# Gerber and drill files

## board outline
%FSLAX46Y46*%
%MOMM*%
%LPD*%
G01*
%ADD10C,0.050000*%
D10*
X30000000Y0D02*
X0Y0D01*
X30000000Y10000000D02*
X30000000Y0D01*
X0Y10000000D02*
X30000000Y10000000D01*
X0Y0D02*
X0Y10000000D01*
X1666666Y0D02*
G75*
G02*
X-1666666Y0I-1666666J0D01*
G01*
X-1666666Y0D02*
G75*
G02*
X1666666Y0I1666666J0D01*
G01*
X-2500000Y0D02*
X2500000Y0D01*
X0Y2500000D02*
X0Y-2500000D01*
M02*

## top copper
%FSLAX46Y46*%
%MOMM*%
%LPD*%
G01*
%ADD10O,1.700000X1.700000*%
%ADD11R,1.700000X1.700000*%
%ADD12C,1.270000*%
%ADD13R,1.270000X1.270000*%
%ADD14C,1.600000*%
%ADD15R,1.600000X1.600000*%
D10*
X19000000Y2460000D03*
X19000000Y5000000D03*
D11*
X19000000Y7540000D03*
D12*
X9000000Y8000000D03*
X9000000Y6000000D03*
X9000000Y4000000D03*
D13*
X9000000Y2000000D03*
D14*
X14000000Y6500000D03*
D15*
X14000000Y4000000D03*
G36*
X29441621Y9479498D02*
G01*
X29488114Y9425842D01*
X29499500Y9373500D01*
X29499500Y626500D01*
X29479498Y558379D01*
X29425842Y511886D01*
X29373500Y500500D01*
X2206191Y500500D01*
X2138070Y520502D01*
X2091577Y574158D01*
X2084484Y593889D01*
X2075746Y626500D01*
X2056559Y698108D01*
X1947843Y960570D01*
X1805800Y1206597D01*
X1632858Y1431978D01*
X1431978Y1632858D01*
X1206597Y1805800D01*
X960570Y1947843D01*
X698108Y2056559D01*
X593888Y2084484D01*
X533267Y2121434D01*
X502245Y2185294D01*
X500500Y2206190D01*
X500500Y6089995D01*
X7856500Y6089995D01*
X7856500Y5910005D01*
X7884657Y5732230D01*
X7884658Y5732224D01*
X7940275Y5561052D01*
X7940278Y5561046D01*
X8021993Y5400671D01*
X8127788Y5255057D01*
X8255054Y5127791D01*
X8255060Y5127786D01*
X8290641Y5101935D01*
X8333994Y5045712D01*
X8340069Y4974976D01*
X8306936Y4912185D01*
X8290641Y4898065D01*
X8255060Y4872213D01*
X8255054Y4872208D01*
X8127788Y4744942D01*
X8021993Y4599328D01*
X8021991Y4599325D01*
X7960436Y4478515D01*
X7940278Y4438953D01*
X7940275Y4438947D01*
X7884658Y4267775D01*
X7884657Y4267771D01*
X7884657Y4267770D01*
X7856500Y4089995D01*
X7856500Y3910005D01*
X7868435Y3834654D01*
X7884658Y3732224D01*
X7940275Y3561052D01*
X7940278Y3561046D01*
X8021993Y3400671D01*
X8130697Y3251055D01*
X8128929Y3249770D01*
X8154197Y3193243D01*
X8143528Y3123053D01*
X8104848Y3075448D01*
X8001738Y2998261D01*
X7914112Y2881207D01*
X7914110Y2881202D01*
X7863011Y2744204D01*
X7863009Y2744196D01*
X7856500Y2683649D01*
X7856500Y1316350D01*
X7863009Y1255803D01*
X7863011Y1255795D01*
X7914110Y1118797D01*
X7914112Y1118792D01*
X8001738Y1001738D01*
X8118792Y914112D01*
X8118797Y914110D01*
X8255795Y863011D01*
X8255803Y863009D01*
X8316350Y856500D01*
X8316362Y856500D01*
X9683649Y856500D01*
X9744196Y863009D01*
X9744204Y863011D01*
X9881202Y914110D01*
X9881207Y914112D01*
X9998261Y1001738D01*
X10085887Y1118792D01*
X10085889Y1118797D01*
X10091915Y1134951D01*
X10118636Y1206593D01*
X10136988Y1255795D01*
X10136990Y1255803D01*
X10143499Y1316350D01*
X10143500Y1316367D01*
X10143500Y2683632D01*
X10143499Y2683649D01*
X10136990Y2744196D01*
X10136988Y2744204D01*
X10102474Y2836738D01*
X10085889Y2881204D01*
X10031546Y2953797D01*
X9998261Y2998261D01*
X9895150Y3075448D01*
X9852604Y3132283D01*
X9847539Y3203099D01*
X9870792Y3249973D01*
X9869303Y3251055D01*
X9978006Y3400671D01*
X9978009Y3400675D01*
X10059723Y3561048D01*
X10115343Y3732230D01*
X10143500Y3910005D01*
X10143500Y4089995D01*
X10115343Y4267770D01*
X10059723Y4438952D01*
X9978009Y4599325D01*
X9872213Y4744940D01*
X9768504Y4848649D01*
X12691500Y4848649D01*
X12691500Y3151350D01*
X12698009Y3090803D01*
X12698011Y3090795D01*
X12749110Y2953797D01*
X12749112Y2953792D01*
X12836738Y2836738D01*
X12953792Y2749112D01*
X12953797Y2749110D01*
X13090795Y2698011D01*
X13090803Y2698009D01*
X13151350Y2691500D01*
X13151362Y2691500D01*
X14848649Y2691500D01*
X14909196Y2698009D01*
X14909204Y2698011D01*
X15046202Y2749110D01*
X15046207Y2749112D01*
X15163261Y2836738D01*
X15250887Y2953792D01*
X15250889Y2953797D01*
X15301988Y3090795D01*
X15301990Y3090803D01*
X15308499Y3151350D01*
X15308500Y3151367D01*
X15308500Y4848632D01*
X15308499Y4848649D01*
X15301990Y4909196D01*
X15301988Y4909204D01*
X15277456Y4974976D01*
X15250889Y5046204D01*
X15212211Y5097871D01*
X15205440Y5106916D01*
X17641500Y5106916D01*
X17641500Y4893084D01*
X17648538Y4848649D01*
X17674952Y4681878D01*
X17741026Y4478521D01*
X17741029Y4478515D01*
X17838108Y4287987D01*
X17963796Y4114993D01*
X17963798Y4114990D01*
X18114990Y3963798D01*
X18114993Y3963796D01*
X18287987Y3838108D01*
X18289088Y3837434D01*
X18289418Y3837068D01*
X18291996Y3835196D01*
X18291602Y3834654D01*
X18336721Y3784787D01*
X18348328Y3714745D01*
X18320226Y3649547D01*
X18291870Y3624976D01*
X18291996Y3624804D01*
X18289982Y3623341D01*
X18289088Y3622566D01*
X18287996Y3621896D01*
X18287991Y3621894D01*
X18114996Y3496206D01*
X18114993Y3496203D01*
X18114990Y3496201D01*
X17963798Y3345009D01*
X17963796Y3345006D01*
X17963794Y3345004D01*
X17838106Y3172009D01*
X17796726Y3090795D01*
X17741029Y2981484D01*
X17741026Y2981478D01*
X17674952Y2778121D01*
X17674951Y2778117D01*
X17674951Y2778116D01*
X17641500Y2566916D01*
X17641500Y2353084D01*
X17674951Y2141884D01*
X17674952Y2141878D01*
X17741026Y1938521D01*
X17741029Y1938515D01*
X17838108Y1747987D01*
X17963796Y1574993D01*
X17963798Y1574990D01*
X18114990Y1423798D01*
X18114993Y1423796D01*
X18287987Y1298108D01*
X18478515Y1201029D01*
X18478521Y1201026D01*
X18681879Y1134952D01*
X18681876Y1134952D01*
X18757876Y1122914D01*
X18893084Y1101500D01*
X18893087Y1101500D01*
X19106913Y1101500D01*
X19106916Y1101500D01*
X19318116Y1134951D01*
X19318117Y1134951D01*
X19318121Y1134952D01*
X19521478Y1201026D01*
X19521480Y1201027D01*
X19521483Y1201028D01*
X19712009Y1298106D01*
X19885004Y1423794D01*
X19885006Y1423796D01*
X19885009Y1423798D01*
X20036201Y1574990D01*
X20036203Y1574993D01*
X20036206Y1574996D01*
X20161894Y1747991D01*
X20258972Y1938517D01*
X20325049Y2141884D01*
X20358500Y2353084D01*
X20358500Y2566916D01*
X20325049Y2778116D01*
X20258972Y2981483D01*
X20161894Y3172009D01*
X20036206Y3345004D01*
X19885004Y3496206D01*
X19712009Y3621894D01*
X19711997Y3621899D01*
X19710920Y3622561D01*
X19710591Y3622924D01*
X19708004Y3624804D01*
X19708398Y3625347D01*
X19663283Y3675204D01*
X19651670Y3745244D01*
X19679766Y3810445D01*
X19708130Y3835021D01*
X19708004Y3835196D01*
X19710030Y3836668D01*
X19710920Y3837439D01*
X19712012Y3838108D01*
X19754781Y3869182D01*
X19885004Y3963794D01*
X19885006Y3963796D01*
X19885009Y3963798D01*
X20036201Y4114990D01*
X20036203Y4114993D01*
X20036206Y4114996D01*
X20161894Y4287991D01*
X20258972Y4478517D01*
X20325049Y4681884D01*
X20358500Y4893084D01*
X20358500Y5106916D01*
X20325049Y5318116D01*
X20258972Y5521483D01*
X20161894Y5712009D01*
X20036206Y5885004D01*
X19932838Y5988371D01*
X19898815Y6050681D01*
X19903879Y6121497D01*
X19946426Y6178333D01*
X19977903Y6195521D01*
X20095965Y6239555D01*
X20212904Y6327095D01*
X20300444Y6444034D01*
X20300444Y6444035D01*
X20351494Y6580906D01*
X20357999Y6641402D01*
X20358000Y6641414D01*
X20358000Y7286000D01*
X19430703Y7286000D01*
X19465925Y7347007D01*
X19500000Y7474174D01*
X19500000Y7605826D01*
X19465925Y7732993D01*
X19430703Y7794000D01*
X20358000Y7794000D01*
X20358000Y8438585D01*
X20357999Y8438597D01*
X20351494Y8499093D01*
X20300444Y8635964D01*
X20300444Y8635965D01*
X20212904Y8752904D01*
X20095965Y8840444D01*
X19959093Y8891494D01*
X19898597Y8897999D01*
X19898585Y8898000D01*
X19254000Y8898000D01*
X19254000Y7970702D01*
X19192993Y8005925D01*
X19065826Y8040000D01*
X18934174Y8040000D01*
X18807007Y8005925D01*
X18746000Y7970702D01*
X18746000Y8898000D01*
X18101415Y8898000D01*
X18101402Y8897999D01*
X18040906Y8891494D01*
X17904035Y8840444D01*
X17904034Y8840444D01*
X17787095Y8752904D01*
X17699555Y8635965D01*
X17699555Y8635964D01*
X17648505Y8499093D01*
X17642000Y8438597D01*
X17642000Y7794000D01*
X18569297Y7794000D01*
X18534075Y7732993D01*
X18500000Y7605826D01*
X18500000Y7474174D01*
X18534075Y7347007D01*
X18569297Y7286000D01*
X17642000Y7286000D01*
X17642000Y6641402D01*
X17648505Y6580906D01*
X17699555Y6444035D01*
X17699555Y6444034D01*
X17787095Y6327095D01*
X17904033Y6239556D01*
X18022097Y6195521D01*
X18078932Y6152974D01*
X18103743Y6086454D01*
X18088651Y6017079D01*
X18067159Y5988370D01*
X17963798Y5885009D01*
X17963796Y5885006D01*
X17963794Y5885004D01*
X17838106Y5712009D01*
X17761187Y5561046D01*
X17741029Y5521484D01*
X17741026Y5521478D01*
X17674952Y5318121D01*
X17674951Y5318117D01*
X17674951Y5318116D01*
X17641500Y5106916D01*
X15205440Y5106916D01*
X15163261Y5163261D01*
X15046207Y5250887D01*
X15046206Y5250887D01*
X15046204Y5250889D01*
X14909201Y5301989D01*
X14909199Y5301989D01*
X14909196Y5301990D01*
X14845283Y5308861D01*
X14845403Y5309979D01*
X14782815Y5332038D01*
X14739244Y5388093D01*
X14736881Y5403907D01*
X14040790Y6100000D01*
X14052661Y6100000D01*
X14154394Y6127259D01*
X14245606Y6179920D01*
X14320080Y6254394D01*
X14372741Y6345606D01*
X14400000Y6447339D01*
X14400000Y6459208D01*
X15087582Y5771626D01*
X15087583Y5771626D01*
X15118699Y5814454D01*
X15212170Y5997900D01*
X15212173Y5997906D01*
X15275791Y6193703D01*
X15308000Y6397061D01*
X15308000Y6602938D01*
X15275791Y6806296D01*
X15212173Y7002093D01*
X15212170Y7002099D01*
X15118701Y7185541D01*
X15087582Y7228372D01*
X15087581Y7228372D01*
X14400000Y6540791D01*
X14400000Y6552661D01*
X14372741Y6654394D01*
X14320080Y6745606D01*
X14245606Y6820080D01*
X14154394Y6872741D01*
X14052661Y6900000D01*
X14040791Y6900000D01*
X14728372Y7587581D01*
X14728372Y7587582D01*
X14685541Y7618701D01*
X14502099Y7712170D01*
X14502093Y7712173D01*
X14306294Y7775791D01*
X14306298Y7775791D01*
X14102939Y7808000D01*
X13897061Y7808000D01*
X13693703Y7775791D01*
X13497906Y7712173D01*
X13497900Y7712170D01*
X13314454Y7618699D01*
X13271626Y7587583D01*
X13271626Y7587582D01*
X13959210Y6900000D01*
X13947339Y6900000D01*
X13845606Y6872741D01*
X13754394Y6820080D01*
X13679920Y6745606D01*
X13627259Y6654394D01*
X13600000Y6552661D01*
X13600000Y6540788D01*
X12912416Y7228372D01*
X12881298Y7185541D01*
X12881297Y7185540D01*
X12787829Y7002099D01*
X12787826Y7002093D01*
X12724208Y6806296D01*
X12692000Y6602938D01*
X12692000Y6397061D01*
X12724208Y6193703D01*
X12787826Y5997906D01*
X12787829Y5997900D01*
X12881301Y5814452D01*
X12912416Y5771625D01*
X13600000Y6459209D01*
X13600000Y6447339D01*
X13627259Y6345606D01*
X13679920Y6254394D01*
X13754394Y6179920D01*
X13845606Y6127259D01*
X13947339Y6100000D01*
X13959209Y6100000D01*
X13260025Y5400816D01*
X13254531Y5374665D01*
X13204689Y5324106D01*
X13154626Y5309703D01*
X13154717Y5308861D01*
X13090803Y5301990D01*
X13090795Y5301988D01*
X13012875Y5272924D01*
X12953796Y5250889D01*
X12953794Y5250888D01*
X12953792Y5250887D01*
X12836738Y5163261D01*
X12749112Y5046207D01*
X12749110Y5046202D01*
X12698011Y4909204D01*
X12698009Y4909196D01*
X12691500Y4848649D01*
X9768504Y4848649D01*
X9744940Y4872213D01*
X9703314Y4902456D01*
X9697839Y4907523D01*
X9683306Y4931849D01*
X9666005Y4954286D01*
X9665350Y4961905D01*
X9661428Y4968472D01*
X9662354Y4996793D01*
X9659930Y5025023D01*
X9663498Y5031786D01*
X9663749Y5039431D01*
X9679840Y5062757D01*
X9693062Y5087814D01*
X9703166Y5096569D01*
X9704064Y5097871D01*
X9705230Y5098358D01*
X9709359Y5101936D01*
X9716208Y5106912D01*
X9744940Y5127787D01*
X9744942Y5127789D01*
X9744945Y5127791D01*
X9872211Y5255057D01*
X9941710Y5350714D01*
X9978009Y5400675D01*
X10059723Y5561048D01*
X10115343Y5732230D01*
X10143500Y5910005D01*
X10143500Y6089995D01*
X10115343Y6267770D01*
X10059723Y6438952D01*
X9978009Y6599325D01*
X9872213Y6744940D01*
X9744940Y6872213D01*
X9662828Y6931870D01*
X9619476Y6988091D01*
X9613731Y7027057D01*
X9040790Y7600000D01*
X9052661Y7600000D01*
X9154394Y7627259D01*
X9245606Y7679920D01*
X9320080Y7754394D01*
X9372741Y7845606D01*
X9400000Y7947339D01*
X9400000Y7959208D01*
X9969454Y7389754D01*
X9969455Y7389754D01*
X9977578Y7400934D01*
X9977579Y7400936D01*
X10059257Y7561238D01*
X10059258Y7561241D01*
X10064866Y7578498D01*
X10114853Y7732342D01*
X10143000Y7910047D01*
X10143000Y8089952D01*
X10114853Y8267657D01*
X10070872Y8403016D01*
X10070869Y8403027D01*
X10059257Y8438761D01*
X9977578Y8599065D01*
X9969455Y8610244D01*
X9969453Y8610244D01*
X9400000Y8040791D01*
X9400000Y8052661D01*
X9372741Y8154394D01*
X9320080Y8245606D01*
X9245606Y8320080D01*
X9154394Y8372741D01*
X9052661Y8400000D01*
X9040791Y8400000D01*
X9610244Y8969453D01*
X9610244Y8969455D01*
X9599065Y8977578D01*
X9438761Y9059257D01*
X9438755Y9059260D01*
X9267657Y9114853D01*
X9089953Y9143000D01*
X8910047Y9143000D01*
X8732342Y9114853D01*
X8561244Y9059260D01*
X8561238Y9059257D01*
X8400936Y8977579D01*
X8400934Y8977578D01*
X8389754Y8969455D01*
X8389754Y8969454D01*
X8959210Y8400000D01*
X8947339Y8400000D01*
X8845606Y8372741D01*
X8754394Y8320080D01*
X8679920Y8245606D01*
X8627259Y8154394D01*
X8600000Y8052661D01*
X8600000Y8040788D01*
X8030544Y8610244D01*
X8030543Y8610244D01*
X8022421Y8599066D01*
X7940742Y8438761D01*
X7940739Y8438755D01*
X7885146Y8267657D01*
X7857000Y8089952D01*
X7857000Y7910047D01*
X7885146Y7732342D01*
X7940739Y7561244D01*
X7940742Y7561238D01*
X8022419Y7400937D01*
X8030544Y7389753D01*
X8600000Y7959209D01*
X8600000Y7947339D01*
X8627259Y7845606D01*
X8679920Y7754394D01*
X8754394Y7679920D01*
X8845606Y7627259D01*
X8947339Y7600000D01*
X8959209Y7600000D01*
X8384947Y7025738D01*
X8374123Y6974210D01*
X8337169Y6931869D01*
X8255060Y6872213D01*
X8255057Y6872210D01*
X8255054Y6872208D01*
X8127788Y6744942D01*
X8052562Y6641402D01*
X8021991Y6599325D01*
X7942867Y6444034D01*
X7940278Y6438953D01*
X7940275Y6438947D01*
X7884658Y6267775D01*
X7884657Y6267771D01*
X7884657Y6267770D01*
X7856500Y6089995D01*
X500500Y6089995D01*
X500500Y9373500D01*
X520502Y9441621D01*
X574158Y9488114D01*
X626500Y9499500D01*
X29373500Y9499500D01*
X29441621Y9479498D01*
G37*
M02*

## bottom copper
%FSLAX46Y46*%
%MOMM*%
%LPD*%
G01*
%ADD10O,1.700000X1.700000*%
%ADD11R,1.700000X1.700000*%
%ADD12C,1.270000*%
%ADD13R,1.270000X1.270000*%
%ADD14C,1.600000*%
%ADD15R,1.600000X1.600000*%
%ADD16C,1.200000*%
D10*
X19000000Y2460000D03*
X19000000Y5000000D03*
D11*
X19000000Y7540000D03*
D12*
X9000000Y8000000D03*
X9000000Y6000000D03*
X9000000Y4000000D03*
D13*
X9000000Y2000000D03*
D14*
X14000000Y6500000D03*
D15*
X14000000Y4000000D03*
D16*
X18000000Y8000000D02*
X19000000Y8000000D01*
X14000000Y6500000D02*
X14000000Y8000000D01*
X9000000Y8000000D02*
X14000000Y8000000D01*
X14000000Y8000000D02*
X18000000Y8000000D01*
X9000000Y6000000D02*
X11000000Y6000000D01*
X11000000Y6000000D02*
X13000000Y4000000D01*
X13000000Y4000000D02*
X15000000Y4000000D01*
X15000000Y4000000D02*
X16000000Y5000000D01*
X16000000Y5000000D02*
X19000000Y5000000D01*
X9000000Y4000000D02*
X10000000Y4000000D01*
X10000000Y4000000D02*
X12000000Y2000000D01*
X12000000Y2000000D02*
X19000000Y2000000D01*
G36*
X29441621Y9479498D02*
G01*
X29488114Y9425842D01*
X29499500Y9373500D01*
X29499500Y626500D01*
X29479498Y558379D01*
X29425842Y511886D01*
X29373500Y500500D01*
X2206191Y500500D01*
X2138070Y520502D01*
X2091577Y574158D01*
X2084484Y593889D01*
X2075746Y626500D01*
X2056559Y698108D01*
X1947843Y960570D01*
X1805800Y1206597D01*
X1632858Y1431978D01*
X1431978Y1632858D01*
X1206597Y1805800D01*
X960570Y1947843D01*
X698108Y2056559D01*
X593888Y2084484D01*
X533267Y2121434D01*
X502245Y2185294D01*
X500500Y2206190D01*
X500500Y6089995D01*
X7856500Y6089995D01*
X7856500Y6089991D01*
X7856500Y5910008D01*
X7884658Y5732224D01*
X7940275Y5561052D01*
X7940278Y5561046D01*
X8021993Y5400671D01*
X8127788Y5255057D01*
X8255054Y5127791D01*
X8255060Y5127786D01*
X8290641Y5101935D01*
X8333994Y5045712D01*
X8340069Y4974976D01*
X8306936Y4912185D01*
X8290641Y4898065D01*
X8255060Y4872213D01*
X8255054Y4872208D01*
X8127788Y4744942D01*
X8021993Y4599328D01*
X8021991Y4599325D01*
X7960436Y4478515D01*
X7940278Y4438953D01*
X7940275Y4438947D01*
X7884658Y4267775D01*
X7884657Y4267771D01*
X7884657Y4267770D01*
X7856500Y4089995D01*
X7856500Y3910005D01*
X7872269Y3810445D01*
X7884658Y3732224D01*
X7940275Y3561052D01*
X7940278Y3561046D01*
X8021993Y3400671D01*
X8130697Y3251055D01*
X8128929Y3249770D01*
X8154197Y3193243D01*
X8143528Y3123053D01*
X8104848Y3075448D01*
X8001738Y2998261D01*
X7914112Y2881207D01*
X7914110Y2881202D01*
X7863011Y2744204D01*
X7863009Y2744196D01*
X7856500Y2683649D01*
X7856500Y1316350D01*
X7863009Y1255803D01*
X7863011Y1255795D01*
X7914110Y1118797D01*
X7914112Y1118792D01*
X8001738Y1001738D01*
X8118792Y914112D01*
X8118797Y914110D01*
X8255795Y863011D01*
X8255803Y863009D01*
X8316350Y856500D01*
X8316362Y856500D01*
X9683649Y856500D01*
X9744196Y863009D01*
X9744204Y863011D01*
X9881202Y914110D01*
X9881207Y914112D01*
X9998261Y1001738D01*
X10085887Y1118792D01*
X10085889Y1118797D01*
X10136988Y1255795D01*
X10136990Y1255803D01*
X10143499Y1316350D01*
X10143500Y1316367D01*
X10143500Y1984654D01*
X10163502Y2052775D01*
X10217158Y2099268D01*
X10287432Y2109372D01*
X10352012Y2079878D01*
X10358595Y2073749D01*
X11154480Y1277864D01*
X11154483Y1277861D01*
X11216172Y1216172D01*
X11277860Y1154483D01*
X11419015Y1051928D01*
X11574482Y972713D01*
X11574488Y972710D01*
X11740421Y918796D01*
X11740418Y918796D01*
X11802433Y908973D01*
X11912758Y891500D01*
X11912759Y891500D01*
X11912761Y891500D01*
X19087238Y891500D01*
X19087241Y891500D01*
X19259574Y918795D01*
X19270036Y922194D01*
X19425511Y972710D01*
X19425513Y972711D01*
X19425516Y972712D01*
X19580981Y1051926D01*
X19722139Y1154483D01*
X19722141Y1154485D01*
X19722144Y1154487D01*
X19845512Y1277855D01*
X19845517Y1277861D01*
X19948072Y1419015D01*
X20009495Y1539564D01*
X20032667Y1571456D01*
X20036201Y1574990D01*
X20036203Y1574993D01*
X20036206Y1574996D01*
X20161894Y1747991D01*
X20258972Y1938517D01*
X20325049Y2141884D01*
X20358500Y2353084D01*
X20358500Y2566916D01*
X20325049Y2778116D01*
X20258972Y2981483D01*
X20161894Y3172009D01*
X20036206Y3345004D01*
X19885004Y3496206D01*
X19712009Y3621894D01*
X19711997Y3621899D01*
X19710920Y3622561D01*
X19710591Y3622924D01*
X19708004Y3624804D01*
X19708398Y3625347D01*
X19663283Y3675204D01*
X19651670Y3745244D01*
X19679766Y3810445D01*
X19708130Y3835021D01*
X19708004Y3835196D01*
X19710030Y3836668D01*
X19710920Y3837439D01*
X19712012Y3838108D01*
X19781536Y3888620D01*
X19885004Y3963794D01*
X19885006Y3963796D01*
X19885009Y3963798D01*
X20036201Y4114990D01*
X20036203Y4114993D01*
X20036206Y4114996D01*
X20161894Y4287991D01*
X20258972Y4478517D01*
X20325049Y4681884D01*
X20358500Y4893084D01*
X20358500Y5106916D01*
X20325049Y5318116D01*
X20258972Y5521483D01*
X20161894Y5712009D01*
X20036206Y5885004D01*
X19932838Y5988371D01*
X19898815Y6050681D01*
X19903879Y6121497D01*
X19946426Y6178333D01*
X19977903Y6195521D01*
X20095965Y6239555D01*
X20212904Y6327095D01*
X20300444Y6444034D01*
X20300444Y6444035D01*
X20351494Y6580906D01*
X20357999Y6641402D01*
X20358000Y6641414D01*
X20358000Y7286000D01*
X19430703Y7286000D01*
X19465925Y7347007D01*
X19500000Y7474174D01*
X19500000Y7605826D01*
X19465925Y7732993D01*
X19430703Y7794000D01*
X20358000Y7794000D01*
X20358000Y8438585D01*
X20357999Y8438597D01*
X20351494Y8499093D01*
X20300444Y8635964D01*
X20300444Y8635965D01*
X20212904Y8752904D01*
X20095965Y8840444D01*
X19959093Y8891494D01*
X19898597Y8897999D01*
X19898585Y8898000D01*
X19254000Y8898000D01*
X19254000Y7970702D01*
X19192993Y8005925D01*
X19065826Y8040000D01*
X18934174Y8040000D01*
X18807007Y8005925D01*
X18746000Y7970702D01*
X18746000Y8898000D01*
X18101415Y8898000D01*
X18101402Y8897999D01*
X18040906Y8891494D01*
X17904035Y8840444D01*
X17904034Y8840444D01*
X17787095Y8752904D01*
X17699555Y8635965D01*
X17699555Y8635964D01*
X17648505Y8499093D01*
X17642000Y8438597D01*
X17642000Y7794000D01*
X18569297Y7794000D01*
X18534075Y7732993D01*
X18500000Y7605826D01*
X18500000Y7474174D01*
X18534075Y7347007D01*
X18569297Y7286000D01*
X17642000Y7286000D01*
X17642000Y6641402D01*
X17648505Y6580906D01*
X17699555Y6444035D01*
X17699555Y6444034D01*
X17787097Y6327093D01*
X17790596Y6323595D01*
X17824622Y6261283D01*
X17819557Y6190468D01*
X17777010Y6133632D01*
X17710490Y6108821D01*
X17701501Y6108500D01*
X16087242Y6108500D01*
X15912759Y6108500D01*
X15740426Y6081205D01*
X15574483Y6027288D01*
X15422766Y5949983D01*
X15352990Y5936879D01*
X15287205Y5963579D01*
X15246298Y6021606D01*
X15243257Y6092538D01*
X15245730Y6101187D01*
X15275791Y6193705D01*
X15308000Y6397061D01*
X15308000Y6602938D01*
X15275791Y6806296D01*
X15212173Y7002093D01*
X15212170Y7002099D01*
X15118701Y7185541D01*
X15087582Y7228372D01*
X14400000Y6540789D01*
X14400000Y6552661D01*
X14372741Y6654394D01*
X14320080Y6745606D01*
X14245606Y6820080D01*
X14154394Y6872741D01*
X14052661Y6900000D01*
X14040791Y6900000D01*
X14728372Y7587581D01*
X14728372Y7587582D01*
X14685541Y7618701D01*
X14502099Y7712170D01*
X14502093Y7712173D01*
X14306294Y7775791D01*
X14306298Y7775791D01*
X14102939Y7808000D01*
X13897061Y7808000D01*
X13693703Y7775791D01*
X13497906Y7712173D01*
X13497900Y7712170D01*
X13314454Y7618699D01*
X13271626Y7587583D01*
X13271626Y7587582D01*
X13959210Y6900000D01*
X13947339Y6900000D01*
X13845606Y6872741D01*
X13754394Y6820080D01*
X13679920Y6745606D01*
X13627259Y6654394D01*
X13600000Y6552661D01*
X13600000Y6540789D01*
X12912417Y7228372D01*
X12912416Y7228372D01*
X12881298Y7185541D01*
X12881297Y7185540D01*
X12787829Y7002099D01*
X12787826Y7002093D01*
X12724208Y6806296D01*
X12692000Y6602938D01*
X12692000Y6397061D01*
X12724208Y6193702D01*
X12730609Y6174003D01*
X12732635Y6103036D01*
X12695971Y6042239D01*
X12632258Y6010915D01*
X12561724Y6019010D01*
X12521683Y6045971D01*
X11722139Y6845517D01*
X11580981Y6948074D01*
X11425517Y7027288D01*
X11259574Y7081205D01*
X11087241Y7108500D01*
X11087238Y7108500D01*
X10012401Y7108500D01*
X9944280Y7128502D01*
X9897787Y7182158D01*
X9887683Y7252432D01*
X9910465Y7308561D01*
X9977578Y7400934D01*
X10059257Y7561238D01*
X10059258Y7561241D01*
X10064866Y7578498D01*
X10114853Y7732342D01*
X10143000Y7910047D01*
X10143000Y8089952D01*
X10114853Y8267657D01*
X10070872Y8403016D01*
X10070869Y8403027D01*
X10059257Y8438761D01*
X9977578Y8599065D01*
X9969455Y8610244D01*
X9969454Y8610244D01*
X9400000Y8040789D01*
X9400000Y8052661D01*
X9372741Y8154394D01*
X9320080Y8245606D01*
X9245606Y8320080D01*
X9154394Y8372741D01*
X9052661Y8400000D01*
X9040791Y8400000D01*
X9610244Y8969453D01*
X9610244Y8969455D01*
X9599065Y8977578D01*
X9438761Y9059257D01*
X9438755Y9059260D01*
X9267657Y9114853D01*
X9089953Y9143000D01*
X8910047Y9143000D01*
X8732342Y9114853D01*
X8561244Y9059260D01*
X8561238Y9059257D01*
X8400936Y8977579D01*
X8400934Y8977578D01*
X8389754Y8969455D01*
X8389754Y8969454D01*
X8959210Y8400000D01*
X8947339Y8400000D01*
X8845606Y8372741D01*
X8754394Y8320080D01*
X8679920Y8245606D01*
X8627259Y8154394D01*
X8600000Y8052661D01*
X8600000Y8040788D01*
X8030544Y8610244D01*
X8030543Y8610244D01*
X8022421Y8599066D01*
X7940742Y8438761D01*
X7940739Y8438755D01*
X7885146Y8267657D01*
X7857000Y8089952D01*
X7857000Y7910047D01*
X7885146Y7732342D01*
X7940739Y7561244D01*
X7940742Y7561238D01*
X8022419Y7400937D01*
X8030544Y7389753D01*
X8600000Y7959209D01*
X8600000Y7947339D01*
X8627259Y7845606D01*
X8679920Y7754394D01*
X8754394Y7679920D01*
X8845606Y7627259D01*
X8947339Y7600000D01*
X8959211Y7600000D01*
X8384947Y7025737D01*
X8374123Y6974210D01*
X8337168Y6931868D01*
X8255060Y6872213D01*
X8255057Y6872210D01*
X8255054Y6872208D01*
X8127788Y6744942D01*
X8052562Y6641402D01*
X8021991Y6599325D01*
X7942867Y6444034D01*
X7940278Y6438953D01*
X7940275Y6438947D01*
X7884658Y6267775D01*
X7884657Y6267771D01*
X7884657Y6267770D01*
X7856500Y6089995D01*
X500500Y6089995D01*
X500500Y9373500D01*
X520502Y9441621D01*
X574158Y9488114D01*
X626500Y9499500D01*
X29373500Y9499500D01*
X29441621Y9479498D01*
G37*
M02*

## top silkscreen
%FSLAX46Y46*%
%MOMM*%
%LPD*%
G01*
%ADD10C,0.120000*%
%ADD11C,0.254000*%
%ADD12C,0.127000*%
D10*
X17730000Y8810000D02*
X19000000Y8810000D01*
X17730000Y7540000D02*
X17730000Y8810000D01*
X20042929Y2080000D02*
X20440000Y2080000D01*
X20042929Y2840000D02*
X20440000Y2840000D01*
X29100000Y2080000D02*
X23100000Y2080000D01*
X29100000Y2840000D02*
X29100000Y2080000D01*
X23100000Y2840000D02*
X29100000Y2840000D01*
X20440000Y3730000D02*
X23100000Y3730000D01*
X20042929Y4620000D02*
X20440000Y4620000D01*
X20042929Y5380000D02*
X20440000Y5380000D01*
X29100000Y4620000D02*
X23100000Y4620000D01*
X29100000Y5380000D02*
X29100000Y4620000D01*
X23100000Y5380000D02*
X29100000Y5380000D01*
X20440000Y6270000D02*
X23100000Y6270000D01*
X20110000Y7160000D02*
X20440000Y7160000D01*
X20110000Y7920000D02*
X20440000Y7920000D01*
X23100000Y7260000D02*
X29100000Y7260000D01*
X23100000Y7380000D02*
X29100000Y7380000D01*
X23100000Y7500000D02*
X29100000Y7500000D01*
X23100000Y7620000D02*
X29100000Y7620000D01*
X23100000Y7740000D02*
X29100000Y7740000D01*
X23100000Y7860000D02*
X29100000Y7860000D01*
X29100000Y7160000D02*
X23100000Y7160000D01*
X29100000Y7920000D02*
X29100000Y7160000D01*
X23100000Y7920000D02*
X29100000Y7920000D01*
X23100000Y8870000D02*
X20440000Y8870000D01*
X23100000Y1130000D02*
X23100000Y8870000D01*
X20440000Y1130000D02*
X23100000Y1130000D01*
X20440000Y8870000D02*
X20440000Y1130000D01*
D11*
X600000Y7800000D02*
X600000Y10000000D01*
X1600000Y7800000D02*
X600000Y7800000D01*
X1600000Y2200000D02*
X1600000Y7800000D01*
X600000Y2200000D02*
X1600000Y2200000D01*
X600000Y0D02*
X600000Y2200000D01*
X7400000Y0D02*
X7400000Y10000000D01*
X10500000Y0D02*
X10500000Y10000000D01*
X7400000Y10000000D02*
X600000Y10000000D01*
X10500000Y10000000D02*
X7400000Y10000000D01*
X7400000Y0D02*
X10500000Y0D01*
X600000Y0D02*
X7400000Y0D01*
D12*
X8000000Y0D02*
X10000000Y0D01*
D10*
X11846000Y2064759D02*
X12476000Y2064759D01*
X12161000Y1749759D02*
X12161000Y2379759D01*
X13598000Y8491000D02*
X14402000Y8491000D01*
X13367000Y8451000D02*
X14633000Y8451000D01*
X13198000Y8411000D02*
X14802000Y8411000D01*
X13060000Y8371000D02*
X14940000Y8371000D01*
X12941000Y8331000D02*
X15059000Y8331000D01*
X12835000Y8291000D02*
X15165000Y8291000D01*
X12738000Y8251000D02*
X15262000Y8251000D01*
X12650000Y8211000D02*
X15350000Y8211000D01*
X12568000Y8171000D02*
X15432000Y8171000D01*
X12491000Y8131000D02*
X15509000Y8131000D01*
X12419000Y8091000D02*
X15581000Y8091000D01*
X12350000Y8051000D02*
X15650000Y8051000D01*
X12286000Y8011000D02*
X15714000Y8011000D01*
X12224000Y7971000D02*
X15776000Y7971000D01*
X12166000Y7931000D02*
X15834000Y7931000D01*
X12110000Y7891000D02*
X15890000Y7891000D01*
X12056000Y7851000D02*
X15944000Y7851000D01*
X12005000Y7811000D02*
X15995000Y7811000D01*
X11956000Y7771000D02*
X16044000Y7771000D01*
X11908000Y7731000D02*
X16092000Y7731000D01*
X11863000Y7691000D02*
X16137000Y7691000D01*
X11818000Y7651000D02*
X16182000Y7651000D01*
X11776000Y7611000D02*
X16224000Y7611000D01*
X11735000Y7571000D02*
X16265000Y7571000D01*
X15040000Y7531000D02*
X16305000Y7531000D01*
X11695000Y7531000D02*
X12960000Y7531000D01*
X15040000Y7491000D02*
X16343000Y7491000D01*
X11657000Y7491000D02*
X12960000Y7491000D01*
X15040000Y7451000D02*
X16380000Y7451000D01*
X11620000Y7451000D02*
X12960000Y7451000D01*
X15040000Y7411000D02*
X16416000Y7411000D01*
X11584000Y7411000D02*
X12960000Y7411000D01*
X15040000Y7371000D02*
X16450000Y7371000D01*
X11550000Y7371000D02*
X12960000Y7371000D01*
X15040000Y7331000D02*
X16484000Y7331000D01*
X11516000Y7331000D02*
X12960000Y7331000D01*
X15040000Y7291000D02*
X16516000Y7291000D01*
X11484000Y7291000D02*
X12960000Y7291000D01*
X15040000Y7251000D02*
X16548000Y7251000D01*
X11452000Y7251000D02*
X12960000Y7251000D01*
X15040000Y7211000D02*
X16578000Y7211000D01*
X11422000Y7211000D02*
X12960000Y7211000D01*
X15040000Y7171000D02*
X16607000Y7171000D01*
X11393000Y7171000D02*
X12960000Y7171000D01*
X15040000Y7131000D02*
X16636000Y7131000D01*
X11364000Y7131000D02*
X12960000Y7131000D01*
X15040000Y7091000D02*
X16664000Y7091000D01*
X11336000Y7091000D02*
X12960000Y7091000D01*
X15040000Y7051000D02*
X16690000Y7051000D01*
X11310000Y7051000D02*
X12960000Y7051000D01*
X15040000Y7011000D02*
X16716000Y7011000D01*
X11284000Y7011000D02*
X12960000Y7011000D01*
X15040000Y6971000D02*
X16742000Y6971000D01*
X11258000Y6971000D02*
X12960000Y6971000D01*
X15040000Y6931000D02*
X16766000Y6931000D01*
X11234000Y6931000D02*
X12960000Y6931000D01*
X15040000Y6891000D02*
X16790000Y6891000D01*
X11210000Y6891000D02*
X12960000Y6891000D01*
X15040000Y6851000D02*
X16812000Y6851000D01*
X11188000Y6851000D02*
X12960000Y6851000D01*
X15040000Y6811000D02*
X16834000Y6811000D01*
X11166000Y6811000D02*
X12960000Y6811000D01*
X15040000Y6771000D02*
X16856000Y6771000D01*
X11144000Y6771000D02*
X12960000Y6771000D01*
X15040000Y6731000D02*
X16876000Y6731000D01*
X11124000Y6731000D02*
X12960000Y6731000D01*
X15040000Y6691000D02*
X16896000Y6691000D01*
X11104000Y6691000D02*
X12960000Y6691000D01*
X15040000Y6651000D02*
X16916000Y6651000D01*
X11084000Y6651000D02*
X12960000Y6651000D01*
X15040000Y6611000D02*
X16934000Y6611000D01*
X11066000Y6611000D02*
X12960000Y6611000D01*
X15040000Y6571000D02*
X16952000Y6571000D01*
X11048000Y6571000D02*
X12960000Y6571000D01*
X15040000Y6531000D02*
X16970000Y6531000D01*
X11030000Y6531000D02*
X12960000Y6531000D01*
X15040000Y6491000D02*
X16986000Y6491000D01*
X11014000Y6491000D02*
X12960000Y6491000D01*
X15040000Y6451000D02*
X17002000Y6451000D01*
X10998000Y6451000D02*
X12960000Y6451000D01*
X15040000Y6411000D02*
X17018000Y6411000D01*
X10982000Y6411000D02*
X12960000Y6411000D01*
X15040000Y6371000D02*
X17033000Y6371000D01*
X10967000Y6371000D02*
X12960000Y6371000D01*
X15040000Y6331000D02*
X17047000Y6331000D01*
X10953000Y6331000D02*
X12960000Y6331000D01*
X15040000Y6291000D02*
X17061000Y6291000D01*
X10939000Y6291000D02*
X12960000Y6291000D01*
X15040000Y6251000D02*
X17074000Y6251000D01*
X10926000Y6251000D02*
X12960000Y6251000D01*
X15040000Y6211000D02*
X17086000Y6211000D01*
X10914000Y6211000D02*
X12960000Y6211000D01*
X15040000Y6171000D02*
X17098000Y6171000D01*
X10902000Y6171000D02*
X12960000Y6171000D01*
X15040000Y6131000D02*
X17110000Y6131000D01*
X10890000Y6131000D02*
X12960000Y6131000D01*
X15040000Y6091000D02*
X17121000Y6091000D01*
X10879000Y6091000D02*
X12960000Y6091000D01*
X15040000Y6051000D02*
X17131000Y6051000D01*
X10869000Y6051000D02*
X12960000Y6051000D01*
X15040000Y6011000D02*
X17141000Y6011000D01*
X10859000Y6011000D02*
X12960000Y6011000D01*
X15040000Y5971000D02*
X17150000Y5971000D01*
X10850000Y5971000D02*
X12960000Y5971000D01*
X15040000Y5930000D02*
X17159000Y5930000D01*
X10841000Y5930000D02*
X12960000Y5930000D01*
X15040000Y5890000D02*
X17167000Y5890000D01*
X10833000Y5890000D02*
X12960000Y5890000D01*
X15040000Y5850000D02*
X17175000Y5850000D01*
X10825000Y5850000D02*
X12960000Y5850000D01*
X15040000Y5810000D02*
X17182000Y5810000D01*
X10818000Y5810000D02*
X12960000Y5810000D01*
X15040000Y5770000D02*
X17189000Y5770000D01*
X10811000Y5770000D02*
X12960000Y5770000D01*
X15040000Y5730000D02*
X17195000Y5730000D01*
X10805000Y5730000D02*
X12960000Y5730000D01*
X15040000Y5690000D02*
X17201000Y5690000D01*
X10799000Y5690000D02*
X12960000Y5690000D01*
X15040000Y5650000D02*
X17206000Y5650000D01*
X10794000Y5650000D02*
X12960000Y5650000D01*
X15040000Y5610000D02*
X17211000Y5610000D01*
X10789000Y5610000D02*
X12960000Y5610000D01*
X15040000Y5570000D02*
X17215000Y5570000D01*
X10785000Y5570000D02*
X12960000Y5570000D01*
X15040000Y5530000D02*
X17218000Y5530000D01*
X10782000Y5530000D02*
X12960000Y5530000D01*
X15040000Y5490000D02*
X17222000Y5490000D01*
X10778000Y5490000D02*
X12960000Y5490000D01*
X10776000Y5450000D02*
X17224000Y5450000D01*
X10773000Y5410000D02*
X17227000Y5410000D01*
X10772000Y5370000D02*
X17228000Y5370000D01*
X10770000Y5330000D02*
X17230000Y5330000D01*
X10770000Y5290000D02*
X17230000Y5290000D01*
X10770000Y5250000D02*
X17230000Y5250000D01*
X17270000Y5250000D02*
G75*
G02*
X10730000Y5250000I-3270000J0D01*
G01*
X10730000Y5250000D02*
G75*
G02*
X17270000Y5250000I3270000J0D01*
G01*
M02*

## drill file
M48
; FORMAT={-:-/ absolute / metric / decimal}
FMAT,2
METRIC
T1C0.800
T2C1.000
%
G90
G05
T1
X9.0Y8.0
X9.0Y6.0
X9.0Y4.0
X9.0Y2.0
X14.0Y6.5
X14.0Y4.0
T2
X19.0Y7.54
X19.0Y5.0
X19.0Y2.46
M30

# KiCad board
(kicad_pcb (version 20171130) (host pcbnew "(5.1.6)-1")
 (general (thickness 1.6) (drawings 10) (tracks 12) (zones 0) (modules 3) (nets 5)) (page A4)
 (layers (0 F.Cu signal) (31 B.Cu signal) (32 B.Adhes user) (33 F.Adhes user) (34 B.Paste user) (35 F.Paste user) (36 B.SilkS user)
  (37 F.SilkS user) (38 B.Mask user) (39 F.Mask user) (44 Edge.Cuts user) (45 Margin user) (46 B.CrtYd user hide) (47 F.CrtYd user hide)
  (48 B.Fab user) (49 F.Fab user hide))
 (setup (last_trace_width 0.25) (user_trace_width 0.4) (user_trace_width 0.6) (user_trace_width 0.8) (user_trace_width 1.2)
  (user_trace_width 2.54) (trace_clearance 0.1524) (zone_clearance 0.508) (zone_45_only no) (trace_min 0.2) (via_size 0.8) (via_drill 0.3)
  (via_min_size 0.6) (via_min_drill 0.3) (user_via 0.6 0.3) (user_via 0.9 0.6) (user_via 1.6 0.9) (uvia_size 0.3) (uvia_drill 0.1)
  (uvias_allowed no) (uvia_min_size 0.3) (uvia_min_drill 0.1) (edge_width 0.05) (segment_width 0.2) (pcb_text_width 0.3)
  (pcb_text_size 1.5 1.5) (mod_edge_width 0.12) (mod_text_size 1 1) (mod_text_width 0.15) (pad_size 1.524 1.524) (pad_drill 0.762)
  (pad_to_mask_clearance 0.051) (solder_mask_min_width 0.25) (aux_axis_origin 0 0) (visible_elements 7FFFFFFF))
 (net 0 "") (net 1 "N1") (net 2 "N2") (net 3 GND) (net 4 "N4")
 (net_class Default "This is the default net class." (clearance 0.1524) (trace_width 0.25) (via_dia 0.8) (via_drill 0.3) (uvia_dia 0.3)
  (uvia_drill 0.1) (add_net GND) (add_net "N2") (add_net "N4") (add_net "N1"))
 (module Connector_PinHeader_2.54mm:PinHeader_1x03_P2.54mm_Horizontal (layer F.Cu) (at 19 -7.54)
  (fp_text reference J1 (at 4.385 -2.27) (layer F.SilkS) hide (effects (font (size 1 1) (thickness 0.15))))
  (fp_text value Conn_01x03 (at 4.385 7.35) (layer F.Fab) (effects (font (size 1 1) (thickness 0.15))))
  (fp_line (start -1.27 -1.27) (end 0 -1.27) (layer F.SilkS) (width 0.12))
  (fp_line (start -1.27 0) (end -1.27 -1.27) (layer F.SilkS) (width 0.12))
  (fp_line (start 1.042929 5.46) (end 1.44 5.46) (layer F.SilkS) (width 0.12))
  (fp_line (start 1.042929 4.7) (end 1.44 4.7) (layer F.SilkS) (width 0.12))
  (fp_line (start 10.1 5.46) (end 4.1 5.46) (layer F.SilkS) (width 0.12))
  (fp_line (start 10.1 4.7) (end 10.1 5.46) (layer F.SilkS) (width 0.12))
  (fp_line (start 4.1 4.7) (end 10.1 4.7) (layer F.SilkS) (width 0.12))
  (fp_line (start 1.44 3.81) (end 4.1 3.81) (layer F.SilkS) (width 0.12))
  (fp_line (start 1.042929 2.92) (end 1.44 2.92) (layer F.SilkS) (width 0.12))
  (fp_line (start 1.042929 2.16) (end 1.44 2.16) (layer F.SilkS) (width 0.12))
  (fp_line (start 10.1 2.92) (end 4.1 2.92) (layer F.SilkS) (width 0.12))
  (fp_line (start 10.1 2.16) (end 10.1 2.92) (layer F.SilkS) (width 0.12))
  (fp_line (start 4.1 2.16) (end 10.1 2.16) (layer F.SilkS) (width 0.12))
  (fp_line (start 1.44 1.27) (end 4.1 1.27) (layer F.SilkS) (width 0.12))
  (fp_line (start 1.11 0.38) (end 1.44 0.38) (layer F.SilkS) (width 0.12))
  (fp_line (start 1.11 -0.38) (end 1.44 -0.38) (layer F.SilkS) (width 0.12))
  (fp_line (start 4.1 0.28) (end 10.1 0.28) (layer F.SilkS) (width 0.12))
  (fp_line (start 4.1 0.16) (end 10.1 0.16) (layer F.SilkS) (width 0.12))
  (fp_line (start 4.1 0.04) (end 10.1 0.04) (layer F.SilkS) (width 0.12))
  (fp_line (start 4.1 -0.08) (end 10.1 -0.08) (layer F.SilkS) (width 0.12))
  (fp_line (start 4.1 -0.2) (end 10.1 -0.2) (layer F.SilkS) (width 0.12))
  (fp_line (start 4.1 -0.32) (end 10.1 -0.32) (layer F.SilkS) (width 0.12))
  (fp_line (start 10.1 0.38) (end 4.1 0.38) (layer F.SilkS) (width 0.12))
  (fp_line (start 10.1 -0.38) (end 10.1 0.38) (layer F.SilkS) (width 0.12))
  (fp_line (start 4.1 -0.38) (end 10.1 -0.38) (layer F.SilkS) (width 0.12))
  (fp_line (start 4.1 -1.33) (end 1.44 -1.33) (layer F.SilkS) (width 0.12))
  (fp_line (start 4.1 6.41) (end 4.1 -1.33) (layer F.SilkS) (width 0.12))
  (fp_line (start 1.44 6.41) (end 4.1 6.41) (layer F.SilkS) (width 0.12))
  (fp_line (start 1.44 -1.33) (end 1.44 6.41) (layer F.SilkS) (width 0.12))
  (pad 3 thru_hole oval (at 0 5.08) (size 1.7 1.7) (drill 1) (layers *.Cu *.Mask) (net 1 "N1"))
  (pad 2 thru_hole oval (at 0 2.54) (size 1.7 1.7) (drill 1) (layers *.Cu *.Mask) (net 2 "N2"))
  (pad 1 thru_hole rect (at 0 0) (size 1.7 1.7) (drill 1) (layers *.Cu *.Mask) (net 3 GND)))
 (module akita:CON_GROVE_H (layer F.Cu) (at 9 -5 90)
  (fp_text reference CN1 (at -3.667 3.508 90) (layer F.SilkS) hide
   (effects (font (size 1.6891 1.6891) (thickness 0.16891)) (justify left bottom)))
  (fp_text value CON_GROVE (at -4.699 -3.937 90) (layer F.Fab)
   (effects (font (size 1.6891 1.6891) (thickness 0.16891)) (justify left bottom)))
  (fp_line (start 2.8 -8.4) (end 5 -8.4) (layer F.SilkS) (width 0.254))
  (fp_line (start 2.8 -7.4) (end 2.8 -8.4) (layer F.SilkS) (width 0.254))
  (fp_line (start -2.8 -7.4) (end 2.8 -7.4) (layer F.SilkS) (width 0.254))
  (fp_line (start -2.8 -8.4) (end -2.8 -7.4) (layer F.SilkS) (width 0.254))
  (fp_line (start -5 -8.4) (end -2.8 -8.4) (layer F.SilkS) (width 0.254))
  (fp_line (start -5 -1.6) (end 5 -1.6) (layer F.SilkS) (width 0.254))
  (fp_line (start -5 1.5) (end 5 1.5) (layer F.SilkS) (width 0.254))
  (fp_line (start 5 -1.6) (end 5 -8.4) (layer F.SilkS) (width 0.254))
  (fp_line (start 5 1.5) (end 5 -1.6) (layer F.SilkS) (width 0.254))
  (fp_line (start -5 -1.6) (end -5 1.5) (layer F.SilkS) (width 0.254))
  (fp_line (start -5 -8.4) (end -5 -1.6) (layer F.SilkS) (width 0.254))
  (fp_line (start -5 -1) (end -5 1) (layer F.SilkS) (width 0.127))
  (pad 4 thru_hole circle (at 3 0 90) (size 1.27 1.27) (drill 0.8) (layers *.Cu *.Mask) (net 3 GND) (solder_mask_margin 0.1016))
  (pad 3 thru_hole circle (at 1 0 90) (size 1.27 1.27) (drill 0.8) (layers *.Cu *.Mask) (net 2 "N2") (solder_mask_margin 0.1016))
  (pad 2 thru_hole circle (at -1 0 90) (size 1.27 1.27) (drill 0.8) (layers *.Cu *.Mask) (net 1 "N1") (solder_mask_margin 0.1016))
  (pad 1 thru_hole rect (at -3 0 90) (size 1.27 1.27) (drill 0.8) (layers *.Cu *.Mask) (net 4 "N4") (solder_mask_margin 0.1016)))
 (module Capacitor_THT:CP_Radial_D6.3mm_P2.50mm (layer F.Cu) (at 14 -4 90)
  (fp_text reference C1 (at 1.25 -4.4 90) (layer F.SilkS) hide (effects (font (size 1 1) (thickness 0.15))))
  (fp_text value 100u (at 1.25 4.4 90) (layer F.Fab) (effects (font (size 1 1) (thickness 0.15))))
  (fp_line (start -1.935241 -2.154) (end -1.935241 -1.524) (layer F.SilkS) (width 0.12))
  (fp_line (start -2.250241 -1.839) (end -1.620241 -1.839) (layer F.SilkS) (width 0.12))
  (fp_line (start 4.491 -0.402) (end 4.491 0.402) (layer F.SilkS) (width 0.12))
  (fp_line (start 4.451 -0.633) (end 4.451 0.633) (layer F.SilkS) (width 0.12))
  (fp_line (start 4.411 -0.802) (end 4.411 0.802) (layer F.SilkS) (width 0.12))
  (fp_line (start 4.371 -0.94) (end 4.371 0.94) (layer F.SilkS) (width 0.12))
  (fp_line (start 4.331 -1.059) (end 4.331 1.059) (layer F.SilkS) (width 0.12))
  (fp_line (start 4.291 -1.165) (end 4.291 1.165) (layer F.SilkS) (width 0.12))
  (fp_line (start 4.251 -1.262) (end 4.251 1.262) (layer F.SilkS) (width 0.12))
  (fp_line (start 4.211 -1.35) (end 4.211 1.35) (layer F.SilkS) (width 0.12))
  (fp_line (start 4.171 -1.432) (end 4.171 1.432) (layer F.SilkS) (width 0.12))
  (fp_line (start 4.131 -1.509) (end 4.131 1.509) (layer F.SilkS) (width 0.12))
  (fp_line (start 4.091 -1.581) (end 4.091 1.581) (layer F.SilkS) (width 0.12))
  (fp_line (start 4.051 -1.65) (end 4.051 1.65) (layer F.SilkS) (width 0.12))
  (fp_line (start 4.011 -1.714) (end 4.011 1.714) (layer F.SilkS) (width 0.12))
  (fp_line (start 3.971 -1.776) (end 3.971 1.776) (layer F.SilkS) (width 0.12))
  (fp_line (start 3.931 -1.834) (end 3.931 1.834) (layer F.SilkS) (width 0.12))
  (fp_line (start 3.891 -1.89) (end 3.891 1.89) (layer F.SilkS) (width 0.12))
  (fp_line (start 3.851 -1.944) (end 3.851 1.944) (layer F.SilkS) (width 0.12))
  (fp_line (start 3.811 -1.995) (end 3.811 1.995) (layer F.SilkS) (width 0.12))
  (fp_line (start 3.771 -2.044) (end 3.771 2.044) (layer F.SilkS) (width 0.12))
  (fp_line (start 3.731 -2.092) (end 3.731 2.092) (layer F.SilkS) (width 0.12))
  (fp_line (start 3.691 -2.137) (end 3.691 2.137) (layer F.SilkS) (width 0.12))
  (fp_line (start 3.651 -2.182) (end 3.651 2.182) (layer F.SilkS) (width 0.12))
  (fp_line (start 3.611 -2.224) (end 3.611 2.224) (layer F.SilkS) (width 0.12))
  (fp_line (start 3.571 -2.265) (end 3.571 2.265) (layer F.SilkS) (width 0.12))
  (fp_line (start 3.531 1.04) (end 3.531 2.305) (layer F.SilkS) (width 0.12))
  (fp_line (start 3.531 -2.305) (end 3.531 -1.04) (layer F.SilkS) (width 0.12))
  (fp_line (start 3.491 1.04) (end 3.491 2.343) (layer F.SilkS) (width 0.12))
  (fp_line (start 3.491 -2.343) (end 3.491 -1.04) (layer F.SilkS) (width 0.12))
  (fp_line (start 3.451 1.04) (end 3.451 2.38) (layer F.SilkS) (width 0.12))
  (fp_line (start 3.451 -2.38) (end 3.451 -1.04) (layer F.SilkS) (width 0.12))
  (fp_line (start 3.411 1.04) (end 3.411 2.416) (layer F.SilkS) (width 0.12))
  (fp_line (start 3.411 -2.416) (end 3.411 -1.04) (layer F.SilkS) (width 0.12))
  (fp_line (start 3.371 1.04) (end 3.371 2.45) (layer F.SilkS) (width 0.12))
  (fp_line (start 3.371 -2.45) (end 3.371 -1.04) (layer F.SilkS) (width 0.12))
  (fp_line (start 3.331 1.04) (end 3.331 2.484) (layer F.SilkS) (width 0.12))
  (fp_line (start 3.331 -2.484) (end 3.331 -1.04) (layer F.SilkS) (width 0.12))
  (fp_line (start 3.291 1.04) (end 3.291 2.516) (layer F.SilkS) (width 0.12))
  (fp_line (start 3.291 -2.516) (end 3.291 -1.04) (layer F.SilkS) (width 0.12))
  (fp_line (start 3.251 1.04) (end 3.251 2.548) (layer F.SilkS) (width 0.12))
  (fp_line (start 3.251 -2.548) (end 3.251 -1.04) (layer F.SilkS) (width 0.12))
  (fp_line (start 3.211 1.04) (end 3.211 2.578) (layer F.SilkS) (width 0.12))
  (fp_line (start 3.211 -2.578) (end 3.211 -1.04) (layer F.SilkS) (width 0.12))
  (fp_line (start 3.171 1.04) (end 3.171 2.607) (layer F.SilkS) (width 0.12))
  (fp_line (start 3.171 -2.607) (end 3.171 -1.04) (layer F.SilkS) (width 0.12))
  (fp_line (start 3.131 1.04) (end 3.131 2.636) (layer F.SilkS) (width 0.12))
  (fp_line (start 3.131 -2.636) (end 3.131 -1.04) (layer F.SilkS) (width 0.12))
  (fp_line (start 3.091 1.04) (end 3.091 2.664) (layer F.SilkS) (width 0.12))
  (fp_line (start 3.091 -2.664) (end 3.091 -1.04) (layer F.SilkS) (width 0.12))
  (fp_line (start 3.051 1.04) (end 3.051 2.69) (layer F.SilkS) (width 0.12))
  (fp_line (start 3.051 -2.69) (end 3.051 -1.04) (layer F.SilkS) (width 0.12))
  (fp_line (start 3.011 1.04) (end 3.011 2.716) (layer F.SilkS) (width 0.12))
  (fp_line (start 3.011 -2.716) (end 3.011 -1.04) (layer F.SilkS) (width 0.12))
  (fp_line (start 2.971 1.04) (end 2.971 2.742) (layer F.SilkS) (width 0.12))
  (fp_line (start 2.971 -2.742) (end 2.971 -1.04) (layer F.SilkS) (width 0.12))
  (fp_line (start 2.931 1.04) (end 2.931 2.766) (layer F.SilkS) (width 0.12))
  (fp_line (start 2.931 -2.766) (end 2.931 -1.04) (layer F.SilkS) (width 0.12))
  (fp_line (start 2.891 1.04) (end 2.891 2.79) (layer F.SilkS) (width 0.12))
  (fp_line (start 2.891 -2.79) (end 2.891 -1.04) (layer F.SilkS) (width 0.12))
  (fp_line (start 2.851 1.04) (end 2.851 2.812) (layer F.SilkS) (width 0.12))
  (fp_line (start 2.851 -2.812) (end 2.851 -1.04) (layer F.SilkS) (width 0.12))
  (fp_line (start 2.811 1.04) (end 2.811 2.834) (layer F.SilkS) (width 0.12))
  (fp_line (start 2.811 -2.834) (end 2.811 -1.04) (layer F.SilkS) (width 0.12))
  (fp_line (start 2.771 1.04) (end 2.771 2.856) (layer F.SilkS) (width 0.12))
  (fp_line (start 2.771 -2.856) (end 2.771 -1.04) (layer F.SilkS) (width 0.12))
  (fp_line (start 2.731 1.04) (end 2.731 2.876) (layer F.SilkS) (width 0.12))
  (fp_line (start 2.731 -2.876) (end 2.731 -1.04) (layer F.SilkS) (width 0.12))
  (fp_line (start 2.691 1.04) (end 2.691 2.896) (layer F.SilkS) (width 0.12))
  (fp_line (start 2.691 -2.896) (end 2.691 -1.04) (layer F.SilkS) (width 0.12))
  (fp_line (start 2.651 1.04) (end 2.651 2.916) (layer F.SilkS) (width 0.12))
  (fp_line (start 2.651 -2.916) (end 2.651 -1.04) (layer F.SilkS) (width 0.12))
  (fp_line (start 2.611 1.04) (end 2.611 2.934) (layer F.SilkS) (width 0.12))
  (fp_line (start 2.611 -2.934) (end 2.611 -1.04) (layer F.SilkS) (width 0.12))
  (fp_line (start 2.571 1.04) (end 2.571 2.952) (layer F.SilkS) (width 0.12))
  (fp_line (start 2.571 -2.952) (end 2.571 -1.04) (layer F.SilkS) (width 0.12))
  (fp_line (start 2.531 1.04) (end 2.531 2.97) (layer F.SilkS) (width 0.12))
  (fp_line (start 2.531 -2.97) (end 2.531 -1.04) (layer F.SilkS) (width 0.12))
  (fp_line (start 2.491 1.04) (end 2.491 2.986) (layer F.SilkS) (width 0.12))
  (fp_line (start 2.491 -2.986) (end 2.491 -1.04) (layer F.SilkS) (width 0.12))
  (fp_line (start 2.451 1.04) (end 2.451 3.002) (layer F.SilkS) (width 0.12))
  (fp_line (start 2.451 -3.002) (end 2.451 -1.04) (layer F.SilkS) (width 0.12))
  (fp_line (start 2.411 1.04) (end 2.411 3.018) (layer F.SilkS) (width 0.12))
  (fp_line (start 2.411 -3.018) (end 2.411 -1.04) (layer F.SilkS) (width 0.12))
  (fp_line (start 2.371 1.04) (end 2.371 3.033) (layer F.SilkS) (width 0.12))
  (fp_line (start 2.371 -3.033) (end 2.371 -1.04) (layer F.SilkS) (width 0.12))
  (fp_line (start 2.331 1.04) (end 2.331 3.047) (layer F.SilkS) (width 0.12))
  (fp_line (start 2.331 -3.047) (end 2.331 -1.04) (layer F.SilkS) (width 0.12))
  (fp_line (start 2.291 1.04) (end 2.291 3.061) (layer F.SilkS) (width 0.12))
  (fp_line (start 2.291 -3.061) (end 2.291 -1.04) (layer F.SilkS) (width 0.12))
  (fp_line (start 2.251 1.04) (end 2.251 3.074) (layer F.SilkS) (width 0.12))
  (fp_line (start 2.251 -3.074) (end 2.251 -1.04) (layer F.SilkS) (width 0.12))
  (fp_line (start 2.211 1.04) (end 2.211 3.086) (layer F.SilkS) (width 0.12))
  (fp_line (start 2.211 -3.086) (end 2.211 -1.04) (layer F.SilkS) (width 0.12))
  (fp_line (start 2.171 1.04) (end 2.171 3.098) (layer F.SilkS) (width 0.12))
  (fp_line (start 2.171 -3.098) (end 2.171 -1.04) (layer F.SilkS) (width 0.12))
  (fp_line (start 2.131 1.04) (end 2.131 3.11) (layer F.SilkS) (width 0.12))
  (fp_line (start 2.131 -3.11) (end 2.131 -1.04) (layer F.SilkS) (width 0.12))
  (fp_line (start 2.091 1.04) (end 2.091 3.121) (layer F.SilkS) (width 0.12))
  (fp_line (start 2.091 -3.121) (end 2.091 -1.04) (layer F.SilkS) (width 0.12))
  (fp_line (start 2.051 1.04) (end 2.051 3.131) (layer F.SilkS) (width 0.12))
  (fp_line (start 2.051 -3.131) (end 2.051 -1.04) (layer F.SilkS) (width 0.12))
  (fp_line (start 2.011 1.04) (end 2.011 3.141) (layer F.SilkS) (width 0.12))
  (fp_line (start 2.011 -3.141) (end 2.011 -1.04) (layer F.SilkS) (width 0.12))
  (fp_line (start 1.971 1.04) (end 1.971 3.15) (layer F.SilkS) (width 0.12))
  (fp_line (start 1.971 -3.15) (end 1.971 -1.04) (layer F.SilkS) (width 0.12))
  (fp_line (start 1.93 1.04) (end 1.93 3.159) (layer F.SilkS) (width 0.12))
  (fp_line (start 1.93 -3.159) (end 1.93 -1.04) (layer F.SilkS) (width 0.12))
  (fp_line (start 1.89 1.04) (end 1.89 3.167) (layer F.SilkS) (width 0.12))
  (fp_line (start 1.89 -3.167) (end 1.89 -1.04) (layer F.SilkS) (width 0.12))
  (fp_line (start 1.85 1.04) (end 1.85 3.175) (layer F.SilkS) (width 0.12))
  (fp_line (start 1.85 -3.175) (end 1.85 -1.04) (layer F.SilkS) (width 0.12))
  (fp_line (start 1.81 1.04) (end 1.81 3.182) (layer F.SilkS) (width 0.12))
  (fp_line (start 1.81 -3.182) (end 1.81 -1.04) (layer F.SilkS) (width 0.12))
  (fp_line (start 1.77 1.04) (end 1.77 3.189) (layer F.SilkS) (width 0.12))
  (fp_line (start 1.77 -3.189) (end 1.77 -1.04) (layer F.SilkS) (width 0.12))
  (fp_line (start 1.73 1.04) (end 1.73 3.195) (layer F.SilkS) (width 0.12))
  (fp_line (start 1.73 -3.195) (end 1.73 -1.04) (layer F.SilkS) (width 0.12))
  (fp_line (start 1.69 1.04) (end 1.69 3.201) (layer F.SilkS) (width 0.12))
  (fp_line (start 1.69 -3.201) (end 1.69 -1.04) (layer F.SilkS) (width 0.12))
  (fp_line (start 1.65 1.04) (end 1.65 3.206) (layer F.SilkS) (width 0.12))
  (fp_line (start 1.65 -3.206) (end 1.65 -1.04) (layer F.SilkS) (width 0.12))
  (fp_line (start 1.61 1.04) (end 1.61 3.211) (layer F.SilkS) (width 0.12))
  (fp_line (start 1.61 -3.211) (end 1.61 -1.04) (layer F.SilkS) (width 0.12))
  (fp_line (start 1.57 1.04) (end 1.57 3.215) (layer F.SilkS) (width 0.12))
  (fp_line (start 1.57 -3.215) (end 1.57 -1.04) (layer F.SilkS) (width 0.12))
  (fp_line (start 1.53 1.04) (end 1.53 3.218) (layer F.SilkS) (width 0.12))
  (fp_line (start 1.53 -3.218) (end 1.53 -1.04) (layer F.SilkS) (width 0.12))
  (fp_line (start 1.49 1.04) (end 1.49 3.222) (layer F.SilkS) (width 0.12))
  (fp_line (start 1.49 -3.222) (end 1.49 -1.04) (layer F.SilkS) (width 0.12))
  (fp_line (start 1.45 -3.224) (end 1.45 3.224) (layer F.SilkS) (width 0.12))
  (fp_line (start 1.41 -3.227) (end 1.41 3.227) (layer F.SilkS) (width 0.12))
  (fp_line (start 1.37 -3.228) (end 1.37 3.228) (layer F.SilkS) (width 0.12))
  (fp_line (start 1.33 -3.23) (end 1.33 3.23) (layer F.SilkS) (width 0.12))
  (fp_line (start 1.29 -3.23) (end 1.29 3.23) (layer F.SilkS) (width 0.12))
  (fp_line (start 1.25 -3.23) (end 1.25 3.23) (layer F.SilkS) (width 0.12))
  (fp_circle (center 1.25 0) (end 4.52 0) (layer F.SilkS) (width 0.12))
  (pad 2 thru_hole circle (at 2.5 0 90) (size 1.6 1.6) (drill 0.8) (layers *.Cu *.Mask) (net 3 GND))
  (pad 1 thru_hole rect (at 0 0 90) (size 1.6 1.6) (drill 0.8) (layers *.Cu *.Mask) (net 2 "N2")))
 (gr_line (start 30 0) (end 0 0) (layer Edge.Cuts) (width 0.05))
 (gr_line (start 30 -10) (end 30 0) (layer Edge.Cuts) (width 0.05))
 (gr_line (start 0 -10) (end 30 -10) (layer Edge.Cuts) (width 0.05))
 (gr_line (start 0 0) (end 0 -10) (layer Edge.Cuts) (width 0.05))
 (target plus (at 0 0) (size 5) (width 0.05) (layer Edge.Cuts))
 (segment (start 18 -8) (end 19 -8) (width 1.2) (layer B.Cu) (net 3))
 (segment (start 14 -6.5) (end 14 -8) (width 1.2) (layer B.Cu) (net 3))
 (segment (start 9 -8) (end 14 -8) (width 1.2) (layer B.Cu) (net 3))
 (segment (start 14 -8) (end 18 -8) (width 1.2) (layer B.Cu) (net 3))
 (segment (start 9 -6) (end 11 -6) (width 1.2) (layer B.Cu) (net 2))
 (segment (start 11 -6) (end 13 -4) (width 1.2) (layer B.Cu) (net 2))
 (segment (start 13 -4) (end 15 -4) (width 1.2) (layer B.Cu) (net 2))
 (segment (start 15 -4) (end 16 -5) (width 1.2) (layer B.Cu) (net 2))
 (segment (start 16 -5) (end 19 -5) (width 1.2) (layer B.Cu) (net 2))
 (segment (start 9 -4) (end 10 -4) (width 1.2) (layer B.Cu) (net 1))
 (segment (start 10 -4) (end 12 -2) (width 1.2) (layer B.Cu) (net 1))
 (segment (start 12 -2) (end 19 -2) (width 1.2) (layer B.Cu) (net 1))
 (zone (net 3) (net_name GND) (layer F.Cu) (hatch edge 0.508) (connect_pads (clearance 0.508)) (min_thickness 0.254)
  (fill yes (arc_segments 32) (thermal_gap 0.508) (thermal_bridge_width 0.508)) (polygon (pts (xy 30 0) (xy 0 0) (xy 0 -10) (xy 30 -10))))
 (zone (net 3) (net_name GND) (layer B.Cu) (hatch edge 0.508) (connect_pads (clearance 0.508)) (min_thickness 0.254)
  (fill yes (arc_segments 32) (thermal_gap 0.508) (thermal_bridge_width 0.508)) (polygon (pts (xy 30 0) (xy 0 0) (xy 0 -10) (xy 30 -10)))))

